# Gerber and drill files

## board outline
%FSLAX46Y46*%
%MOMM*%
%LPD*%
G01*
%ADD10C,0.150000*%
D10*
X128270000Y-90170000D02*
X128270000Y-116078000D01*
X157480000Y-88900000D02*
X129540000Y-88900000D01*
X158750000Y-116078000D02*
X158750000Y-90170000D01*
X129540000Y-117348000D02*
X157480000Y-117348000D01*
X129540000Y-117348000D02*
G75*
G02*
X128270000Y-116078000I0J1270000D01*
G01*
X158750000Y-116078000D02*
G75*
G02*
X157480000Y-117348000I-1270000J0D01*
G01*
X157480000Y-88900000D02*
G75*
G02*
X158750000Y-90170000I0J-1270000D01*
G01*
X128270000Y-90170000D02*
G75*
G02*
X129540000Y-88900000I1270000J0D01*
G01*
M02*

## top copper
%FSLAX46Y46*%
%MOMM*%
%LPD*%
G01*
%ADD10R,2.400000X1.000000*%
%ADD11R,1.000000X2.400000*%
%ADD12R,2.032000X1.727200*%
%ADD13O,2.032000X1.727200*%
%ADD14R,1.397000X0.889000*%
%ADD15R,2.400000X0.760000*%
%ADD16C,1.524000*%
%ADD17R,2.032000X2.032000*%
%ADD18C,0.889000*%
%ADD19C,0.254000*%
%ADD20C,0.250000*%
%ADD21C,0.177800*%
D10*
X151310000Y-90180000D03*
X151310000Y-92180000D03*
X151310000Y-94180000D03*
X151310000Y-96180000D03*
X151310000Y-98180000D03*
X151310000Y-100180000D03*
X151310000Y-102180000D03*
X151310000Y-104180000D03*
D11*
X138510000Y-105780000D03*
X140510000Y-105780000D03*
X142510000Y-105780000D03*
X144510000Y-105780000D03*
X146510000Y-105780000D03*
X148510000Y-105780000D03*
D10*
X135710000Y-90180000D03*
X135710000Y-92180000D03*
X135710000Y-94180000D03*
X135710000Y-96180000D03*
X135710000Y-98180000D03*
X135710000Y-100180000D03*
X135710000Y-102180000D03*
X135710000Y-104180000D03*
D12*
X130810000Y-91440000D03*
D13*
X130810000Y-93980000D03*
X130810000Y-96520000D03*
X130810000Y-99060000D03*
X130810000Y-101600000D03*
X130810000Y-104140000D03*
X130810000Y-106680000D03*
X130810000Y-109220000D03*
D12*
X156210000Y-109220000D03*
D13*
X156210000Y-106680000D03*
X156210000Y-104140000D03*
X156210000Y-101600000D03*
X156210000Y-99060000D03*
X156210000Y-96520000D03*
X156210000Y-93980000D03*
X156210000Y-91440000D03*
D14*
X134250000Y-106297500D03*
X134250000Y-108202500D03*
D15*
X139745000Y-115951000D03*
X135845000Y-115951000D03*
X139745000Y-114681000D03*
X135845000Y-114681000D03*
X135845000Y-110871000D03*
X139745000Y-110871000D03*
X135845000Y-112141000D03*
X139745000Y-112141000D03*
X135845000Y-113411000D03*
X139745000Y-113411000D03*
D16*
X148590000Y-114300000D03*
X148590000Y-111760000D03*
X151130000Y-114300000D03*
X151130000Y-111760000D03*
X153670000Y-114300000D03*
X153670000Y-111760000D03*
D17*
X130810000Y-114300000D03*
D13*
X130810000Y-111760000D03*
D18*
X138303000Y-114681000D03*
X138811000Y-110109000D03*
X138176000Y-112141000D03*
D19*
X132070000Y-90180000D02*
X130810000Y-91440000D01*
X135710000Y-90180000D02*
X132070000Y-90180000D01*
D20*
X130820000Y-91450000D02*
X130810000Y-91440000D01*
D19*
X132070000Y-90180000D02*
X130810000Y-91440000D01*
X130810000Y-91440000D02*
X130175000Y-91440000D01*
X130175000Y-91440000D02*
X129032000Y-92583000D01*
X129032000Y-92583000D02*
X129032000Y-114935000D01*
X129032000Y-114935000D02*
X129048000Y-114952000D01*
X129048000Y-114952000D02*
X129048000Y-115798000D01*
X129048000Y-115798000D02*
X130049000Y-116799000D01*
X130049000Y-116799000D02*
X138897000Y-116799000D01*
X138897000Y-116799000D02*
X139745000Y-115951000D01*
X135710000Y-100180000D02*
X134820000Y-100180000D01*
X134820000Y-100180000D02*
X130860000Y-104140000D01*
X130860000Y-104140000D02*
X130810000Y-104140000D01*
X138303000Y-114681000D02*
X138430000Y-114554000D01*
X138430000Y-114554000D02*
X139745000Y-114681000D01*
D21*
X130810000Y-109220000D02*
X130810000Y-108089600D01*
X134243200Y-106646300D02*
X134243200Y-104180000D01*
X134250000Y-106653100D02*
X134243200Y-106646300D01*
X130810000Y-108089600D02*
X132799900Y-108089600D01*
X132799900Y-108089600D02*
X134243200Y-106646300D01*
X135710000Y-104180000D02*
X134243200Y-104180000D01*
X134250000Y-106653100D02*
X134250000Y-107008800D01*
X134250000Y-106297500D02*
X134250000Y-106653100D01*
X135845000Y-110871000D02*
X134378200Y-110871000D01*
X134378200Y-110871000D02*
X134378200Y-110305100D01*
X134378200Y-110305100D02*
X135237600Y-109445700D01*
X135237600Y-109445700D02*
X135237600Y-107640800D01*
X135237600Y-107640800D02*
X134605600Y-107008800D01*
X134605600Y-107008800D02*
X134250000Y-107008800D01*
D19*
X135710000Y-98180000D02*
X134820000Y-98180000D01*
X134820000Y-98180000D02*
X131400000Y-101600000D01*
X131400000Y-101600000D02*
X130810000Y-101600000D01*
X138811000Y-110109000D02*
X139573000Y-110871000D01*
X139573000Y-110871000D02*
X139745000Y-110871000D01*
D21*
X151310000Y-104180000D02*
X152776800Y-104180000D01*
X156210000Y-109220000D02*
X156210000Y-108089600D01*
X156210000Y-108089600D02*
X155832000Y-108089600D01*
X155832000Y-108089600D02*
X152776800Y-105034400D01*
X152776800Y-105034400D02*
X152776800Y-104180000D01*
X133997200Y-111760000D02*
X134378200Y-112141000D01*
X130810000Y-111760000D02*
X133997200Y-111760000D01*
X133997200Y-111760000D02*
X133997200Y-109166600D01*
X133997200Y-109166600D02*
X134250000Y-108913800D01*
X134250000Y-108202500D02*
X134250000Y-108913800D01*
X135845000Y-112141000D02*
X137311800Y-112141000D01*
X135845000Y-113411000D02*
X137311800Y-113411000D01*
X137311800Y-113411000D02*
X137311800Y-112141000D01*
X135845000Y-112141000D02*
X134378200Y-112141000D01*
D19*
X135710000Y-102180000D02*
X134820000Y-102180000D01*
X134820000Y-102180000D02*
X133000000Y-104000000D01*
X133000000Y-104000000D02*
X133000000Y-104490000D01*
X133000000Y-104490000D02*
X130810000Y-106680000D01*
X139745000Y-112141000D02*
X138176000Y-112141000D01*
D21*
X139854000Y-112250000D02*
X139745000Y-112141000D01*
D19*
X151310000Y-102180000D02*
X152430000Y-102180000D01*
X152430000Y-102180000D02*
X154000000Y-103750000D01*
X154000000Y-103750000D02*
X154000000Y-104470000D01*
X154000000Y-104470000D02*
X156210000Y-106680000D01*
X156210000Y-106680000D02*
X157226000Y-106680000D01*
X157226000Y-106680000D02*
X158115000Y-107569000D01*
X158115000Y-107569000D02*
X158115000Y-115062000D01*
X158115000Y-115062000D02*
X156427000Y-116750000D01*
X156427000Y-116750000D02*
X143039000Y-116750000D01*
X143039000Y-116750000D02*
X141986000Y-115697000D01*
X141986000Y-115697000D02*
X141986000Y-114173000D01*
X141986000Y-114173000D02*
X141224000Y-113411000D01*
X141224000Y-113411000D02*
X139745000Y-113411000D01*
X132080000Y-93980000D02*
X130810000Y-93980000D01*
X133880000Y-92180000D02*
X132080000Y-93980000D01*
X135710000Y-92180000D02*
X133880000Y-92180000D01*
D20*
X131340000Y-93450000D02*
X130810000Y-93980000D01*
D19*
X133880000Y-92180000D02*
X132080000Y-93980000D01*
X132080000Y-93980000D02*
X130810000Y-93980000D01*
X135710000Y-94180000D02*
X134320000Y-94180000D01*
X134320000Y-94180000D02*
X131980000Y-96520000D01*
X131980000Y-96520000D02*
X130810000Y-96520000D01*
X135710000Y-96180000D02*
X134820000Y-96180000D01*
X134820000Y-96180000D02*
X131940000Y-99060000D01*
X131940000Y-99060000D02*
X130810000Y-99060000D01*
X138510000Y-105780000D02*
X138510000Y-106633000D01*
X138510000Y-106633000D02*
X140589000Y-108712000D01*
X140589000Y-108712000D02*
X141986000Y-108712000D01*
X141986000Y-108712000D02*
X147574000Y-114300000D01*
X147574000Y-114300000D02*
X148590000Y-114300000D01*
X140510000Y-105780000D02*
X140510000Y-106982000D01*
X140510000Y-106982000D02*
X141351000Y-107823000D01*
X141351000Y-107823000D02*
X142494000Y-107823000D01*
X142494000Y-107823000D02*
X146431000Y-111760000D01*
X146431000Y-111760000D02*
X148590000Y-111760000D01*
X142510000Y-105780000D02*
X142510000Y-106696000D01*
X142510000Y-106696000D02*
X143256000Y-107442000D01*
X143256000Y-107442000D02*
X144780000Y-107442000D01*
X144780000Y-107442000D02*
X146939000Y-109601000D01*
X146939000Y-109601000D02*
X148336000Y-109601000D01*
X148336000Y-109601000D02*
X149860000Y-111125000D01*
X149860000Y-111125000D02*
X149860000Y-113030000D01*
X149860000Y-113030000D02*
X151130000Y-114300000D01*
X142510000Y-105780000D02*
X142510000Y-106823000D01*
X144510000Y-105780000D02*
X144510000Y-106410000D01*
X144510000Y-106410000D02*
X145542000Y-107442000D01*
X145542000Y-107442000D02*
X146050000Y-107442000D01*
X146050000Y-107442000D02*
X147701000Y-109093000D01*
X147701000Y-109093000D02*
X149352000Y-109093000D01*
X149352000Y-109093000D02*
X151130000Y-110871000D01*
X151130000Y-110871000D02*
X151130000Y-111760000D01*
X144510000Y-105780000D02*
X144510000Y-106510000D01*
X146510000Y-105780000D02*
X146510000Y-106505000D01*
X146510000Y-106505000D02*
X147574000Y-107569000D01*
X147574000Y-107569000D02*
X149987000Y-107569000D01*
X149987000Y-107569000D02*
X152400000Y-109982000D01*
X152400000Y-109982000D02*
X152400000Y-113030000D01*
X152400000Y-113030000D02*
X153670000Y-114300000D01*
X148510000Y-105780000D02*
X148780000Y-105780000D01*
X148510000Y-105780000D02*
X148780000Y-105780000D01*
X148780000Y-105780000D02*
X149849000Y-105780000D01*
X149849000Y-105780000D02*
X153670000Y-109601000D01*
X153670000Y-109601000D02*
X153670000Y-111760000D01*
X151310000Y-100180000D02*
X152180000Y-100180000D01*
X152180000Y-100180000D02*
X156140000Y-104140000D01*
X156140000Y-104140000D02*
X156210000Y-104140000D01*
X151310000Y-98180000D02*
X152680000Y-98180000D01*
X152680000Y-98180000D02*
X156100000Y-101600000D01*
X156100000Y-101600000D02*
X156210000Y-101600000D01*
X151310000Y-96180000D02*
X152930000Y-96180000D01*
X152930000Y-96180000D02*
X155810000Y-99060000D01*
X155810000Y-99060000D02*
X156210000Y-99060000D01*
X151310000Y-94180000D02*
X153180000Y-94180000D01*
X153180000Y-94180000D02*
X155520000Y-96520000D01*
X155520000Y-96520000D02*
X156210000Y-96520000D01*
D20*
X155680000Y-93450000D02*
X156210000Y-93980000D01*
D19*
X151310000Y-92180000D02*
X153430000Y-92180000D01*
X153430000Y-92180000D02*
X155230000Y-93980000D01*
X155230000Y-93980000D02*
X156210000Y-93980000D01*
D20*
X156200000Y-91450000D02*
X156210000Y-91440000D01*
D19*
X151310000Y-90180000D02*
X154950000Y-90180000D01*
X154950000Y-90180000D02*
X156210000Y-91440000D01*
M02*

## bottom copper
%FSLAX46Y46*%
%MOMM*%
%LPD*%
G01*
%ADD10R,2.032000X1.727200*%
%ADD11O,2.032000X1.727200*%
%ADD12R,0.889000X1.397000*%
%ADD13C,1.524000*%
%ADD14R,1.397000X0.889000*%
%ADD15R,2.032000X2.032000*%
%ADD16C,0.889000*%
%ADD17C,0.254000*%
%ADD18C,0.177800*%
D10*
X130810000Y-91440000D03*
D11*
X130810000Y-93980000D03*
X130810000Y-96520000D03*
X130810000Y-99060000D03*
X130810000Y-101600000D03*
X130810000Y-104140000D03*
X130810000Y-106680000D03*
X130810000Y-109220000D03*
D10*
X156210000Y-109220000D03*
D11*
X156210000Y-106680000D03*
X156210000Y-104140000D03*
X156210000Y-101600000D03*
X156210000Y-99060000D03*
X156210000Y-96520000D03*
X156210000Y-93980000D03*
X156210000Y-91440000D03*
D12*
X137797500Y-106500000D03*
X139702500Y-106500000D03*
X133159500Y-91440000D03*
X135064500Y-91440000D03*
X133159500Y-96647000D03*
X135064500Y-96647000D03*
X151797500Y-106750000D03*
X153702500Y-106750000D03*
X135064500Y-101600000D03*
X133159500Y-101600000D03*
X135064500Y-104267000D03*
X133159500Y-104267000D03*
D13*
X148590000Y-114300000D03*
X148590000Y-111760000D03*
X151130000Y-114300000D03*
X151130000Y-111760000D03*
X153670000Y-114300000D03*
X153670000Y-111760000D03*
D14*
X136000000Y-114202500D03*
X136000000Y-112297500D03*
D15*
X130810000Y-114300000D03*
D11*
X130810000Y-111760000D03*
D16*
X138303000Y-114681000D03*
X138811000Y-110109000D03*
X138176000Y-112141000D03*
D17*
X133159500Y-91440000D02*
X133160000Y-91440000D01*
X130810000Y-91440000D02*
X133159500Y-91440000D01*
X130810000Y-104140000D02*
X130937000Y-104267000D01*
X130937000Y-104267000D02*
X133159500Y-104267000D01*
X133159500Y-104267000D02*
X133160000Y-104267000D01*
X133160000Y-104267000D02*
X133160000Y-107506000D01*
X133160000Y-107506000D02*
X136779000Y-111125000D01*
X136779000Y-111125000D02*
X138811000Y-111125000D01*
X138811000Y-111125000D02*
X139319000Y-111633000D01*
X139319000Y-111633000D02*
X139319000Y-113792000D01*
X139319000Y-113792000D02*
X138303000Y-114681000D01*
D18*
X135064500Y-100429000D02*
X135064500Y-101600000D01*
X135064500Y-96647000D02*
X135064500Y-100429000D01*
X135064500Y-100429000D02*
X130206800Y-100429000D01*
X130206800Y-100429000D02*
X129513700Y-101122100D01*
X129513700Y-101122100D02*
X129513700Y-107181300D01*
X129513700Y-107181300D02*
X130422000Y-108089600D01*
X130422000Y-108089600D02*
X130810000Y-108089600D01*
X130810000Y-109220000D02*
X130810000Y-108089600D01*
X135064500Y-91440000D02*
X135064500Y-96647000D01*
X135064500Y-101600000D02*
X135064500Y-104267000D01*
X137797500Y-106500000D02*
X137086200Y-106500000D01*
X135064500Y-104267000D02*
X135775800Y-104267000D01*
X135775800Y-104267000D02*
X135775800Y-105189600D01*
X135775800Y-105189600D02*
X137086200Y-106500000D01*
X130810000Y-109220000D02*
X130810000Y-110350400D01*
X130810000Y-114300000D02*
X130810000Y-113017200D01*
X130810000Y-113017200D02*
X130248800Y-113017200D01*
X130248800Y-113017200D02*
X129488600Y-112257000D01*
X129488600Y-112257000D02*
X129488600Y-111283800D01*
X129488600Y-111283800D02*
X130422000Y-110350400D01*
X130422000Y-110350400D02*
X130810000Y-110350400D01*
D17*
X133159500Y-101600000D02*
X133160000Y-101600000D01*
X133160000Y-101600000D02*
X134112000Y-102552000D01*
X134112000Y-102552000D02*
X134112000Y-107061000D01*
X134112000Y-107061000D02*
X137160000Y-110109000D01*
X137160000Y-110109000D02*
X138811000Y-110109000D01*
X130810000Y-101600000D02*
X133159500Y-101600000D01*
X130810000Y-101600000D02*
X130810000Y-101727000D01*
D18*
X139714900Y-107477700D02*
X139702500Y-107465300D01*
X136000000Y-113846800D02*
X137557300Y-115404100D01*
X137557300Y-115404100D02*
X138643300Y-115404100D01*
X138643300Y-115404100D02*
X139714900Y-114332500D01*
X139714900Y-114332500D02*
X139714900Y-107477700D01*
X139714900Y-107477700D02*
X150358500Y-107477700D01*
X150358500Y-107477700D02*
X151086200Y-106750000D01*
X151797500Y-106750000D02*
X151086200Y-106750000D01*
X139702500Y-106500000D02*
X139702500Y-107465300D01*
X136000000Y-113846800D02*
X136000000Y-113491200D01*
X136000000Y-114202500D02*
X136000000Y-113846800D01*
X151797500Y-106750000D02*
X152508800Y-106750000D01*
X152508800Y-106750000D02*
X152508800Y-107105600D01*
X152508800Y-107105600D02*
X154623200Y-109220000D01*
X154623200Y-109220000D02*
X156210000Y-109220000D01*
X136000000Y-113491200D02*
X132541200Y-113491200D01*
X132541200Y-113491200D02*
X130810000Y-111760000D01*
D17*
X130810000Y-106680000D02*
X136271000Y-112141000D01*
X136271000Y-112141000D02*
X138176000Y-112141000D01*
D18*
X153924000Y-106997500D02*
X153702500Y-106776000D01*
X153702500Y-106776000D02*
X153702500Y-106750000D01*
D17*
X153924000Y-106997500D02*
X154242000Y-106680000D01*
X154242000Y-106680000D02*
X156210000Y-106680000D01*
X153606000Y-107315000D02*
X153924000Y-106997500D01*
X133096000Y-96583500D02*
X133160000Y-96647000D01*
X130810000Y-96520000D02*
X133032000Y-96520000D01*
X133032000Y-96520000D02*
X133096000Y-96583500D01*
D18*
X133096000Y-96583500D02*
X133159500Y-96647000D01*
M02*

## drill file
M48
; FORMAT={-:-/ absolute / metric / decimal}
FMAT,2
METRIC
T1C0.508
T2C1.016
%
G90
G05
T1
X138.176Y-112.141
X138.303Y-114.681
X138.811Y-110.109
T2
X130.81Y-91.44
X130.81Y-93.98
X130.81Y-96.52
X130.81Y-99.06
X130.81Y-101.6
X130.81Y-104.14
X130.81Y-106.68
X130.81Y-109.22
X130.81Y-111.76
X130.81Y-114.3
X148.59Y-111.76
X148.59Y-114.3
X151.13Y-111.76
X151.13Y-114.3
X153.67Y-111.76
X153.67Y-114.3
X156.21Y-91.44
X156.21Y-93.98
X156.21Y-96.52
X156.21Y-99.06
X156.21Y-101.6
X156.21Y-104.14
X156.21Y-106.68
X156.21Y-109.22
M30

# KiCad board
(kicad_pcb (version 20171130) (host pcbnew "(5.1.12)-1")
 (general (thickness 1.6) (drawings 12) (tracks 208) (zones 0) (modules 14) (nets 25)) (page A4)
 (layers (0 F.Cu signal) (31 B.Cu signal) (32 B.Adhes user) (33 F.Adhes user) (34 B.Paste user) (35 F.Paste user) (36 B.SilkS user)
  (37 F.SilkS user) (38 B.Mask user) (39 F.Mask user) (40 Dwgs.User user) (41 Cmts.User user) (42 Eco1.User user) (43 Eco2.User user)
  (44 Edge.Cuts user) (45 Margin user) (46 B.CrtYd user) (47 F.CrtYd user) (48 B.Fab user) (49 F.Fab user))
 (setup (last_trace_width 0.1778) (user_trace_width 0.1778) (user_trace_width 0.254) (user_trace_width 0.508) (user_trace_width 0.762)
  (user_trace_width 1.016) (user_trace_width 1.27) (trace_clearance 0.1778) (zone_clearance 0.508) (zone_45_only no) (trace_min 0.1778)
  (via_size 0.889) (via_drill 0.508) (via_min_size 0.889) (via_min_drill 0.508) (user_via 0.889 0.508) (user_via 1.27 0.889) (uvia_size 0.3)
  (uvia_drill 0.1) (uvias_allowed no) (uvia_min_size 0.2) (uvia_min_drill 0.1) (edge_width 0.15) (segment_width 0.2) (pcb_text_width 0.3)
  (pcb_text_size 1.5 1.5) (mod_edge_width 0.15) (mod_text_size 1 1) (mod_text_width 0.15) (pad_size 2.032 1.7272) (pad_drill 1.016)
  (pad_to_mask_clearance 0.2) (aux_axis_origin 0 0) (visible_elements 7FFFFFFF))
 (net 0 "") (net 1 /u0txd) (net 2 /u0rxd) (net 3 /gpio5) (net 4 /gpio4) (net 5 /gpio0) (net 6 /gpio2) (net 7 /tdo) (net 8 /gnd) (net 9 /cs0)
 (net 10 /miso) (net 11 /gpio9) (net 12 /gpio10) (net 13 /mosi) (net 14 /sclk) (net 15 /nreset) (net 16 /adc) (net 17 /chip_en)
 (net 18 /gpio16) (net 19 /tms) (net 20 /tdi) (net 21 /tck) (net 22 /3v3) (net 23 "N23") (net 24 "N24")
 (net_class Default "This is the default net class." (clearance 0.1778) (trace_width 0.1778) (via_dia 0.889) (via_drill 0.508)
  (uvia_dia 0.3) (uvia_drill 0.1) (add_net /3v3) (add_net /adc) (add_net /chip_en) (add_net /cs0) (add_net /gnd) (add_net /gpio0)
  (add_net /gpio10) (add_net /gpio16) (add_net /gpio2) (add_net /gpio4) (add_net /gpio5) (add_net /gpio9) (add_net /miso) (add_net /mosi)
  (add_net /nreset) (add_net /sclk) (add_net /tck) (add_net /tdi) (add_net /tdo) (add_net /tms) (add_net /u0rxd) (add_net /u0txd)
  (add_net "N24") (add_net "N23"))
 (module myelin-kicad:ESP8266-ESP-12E (layer F.Cu) (at 143.51 93.98)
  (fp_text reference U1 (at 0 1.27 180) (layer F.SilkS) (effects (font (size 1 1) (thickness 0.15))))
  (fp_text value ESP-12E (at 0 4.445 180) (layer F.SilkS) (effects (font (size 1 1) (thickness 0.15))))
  (pad 22 smd rect (at 7.8 -3.8) (size 2.4 1) (layers F.Cu F.Paste F.Mask) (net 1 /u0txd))
  (pad 21 smd rect (at 7.8 -1.8) (size 2.4 1) (layers F.Cu F.Paste F.Mask) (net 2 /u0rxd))
  (pad 20 smd rect (at 7.8 0.2) (size 2.4 1) (layers F.Cu F.Paste F.Mask) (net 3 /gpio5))
  (pad 19 smd rect (at 7.8 2.2) (size 2.4 1) (layers F.Cu F.Paste F.Mask) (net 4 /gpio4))
  (pad 18 smd rect (at 7.8 4.2) (size 2.4 1) (layers F.Cu F.Paste F.Mask) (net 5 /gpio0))
  (pad 17 smd rect (at 7.8 6.2) (size 2.4 1) (layers F.Cu F.Paste F.Mask) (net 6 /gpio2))
  (pad 16 smd rect (at 7.8 8.2) (size 2.4 1) (layers F.Cu F.Paste F.Mask) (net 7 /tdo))
  (pad 15 smd rect (at 7.8 10.2) (size 2.4 1) (layers F.Cu F.Paste F.Mask) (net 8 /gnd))
  (pad 9 smd rect (at -5 11.8) (size 1 2.4) (layers F.Cu F.Paste F.Mask) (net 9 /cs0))
  (pad 10 smd rect (at -3 11.8) (size 1 2.4) (layers F.Cu F.Paste F.Mask) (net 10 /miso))
  (pad 11 smd rect (at -1 11.8) (size 1 2.4) (layers F.Cu F.Paste F.Mask) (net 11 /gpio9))
  (pad 12 smd rect (at 1 11.8) (size 1 2.4) (layers F.Cu F.Paste F.Mask) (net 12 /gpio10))
  (pad 13 smd rect (at 3 11.8) (size 1 2.4) (layers F.Cu F.Paste F.Mask) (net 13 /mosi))
  (pad 14 smd rect (at 5 11.8) (size 1 2.4) (layers F.Cu F.Paste F.Mask) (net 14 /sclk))
  (pad 1 smd rect (at -7.8 -3.8) (size 2.4 1) (layers F.Cu F.Paste F.Mask) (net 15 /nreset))
  (pad 2 smd rect (at -7.8 -1.8) (size 2.4 1) (layers F.Cu F.Paste F.Mask) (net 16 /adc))
  (pad 3 smd rect (at -7.8 0.2) (size 2.4 1) (layers F.Cu F.Paste F.Mask) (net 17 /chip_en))
  (pad 4 smd rect (at -7.8 2.2) (size 2.4 1) (layers F.Cu F.Paste F.Mask) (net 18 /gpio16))
  (pad 5 smd rect (at -7.8 4.2) (size 2.4 1) (layers F.Cu F.Paste F.Mask) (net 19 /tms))
  (pad 6 smd rect (at -7.8 6.2) (size 2.4 1) (layers F.Cu F.Paste F.Mask) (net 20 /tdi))
  (pad 7 smd rect (at -7.8 8.2) (size 2.4 1) (layers F.Cu F.Paste F.Mask) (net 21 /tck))
  (pad 8 smd rect (at -7.8 10.2) (size 2.4 1) (layers F.Cu F.Paste F.Mask) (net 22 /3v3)))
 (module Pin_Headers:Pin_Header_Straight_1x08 (layer F.Cu) (at 130.81 91.44)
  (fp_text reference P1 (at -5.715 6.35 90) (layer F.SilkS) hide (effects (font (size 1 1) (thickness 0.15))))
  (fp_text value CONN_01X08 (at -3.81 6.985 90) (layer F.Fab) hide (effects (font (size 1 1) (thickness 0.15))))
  (pad 1 thru_hole rect (at 0 0) (size 2.032 1.7272) (drill 1.016) (layers *.Cu *.Mask F.SilkS) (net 15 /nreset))
  (pad 2 thru_hole oval (at 0 2.54) (size 2.032 1.7272) (drill 1.016) (layers *.Cu *.Mask F.SilkS) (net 16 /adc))
  (pad 3 thru_hole oval (at 0 5.08) (size 2.032 1.7272) (drill 1.016) (layers *.Cu *.Mask F.SilkS) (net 17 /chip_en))
  (pad 4 thru_hole oval (at 0 7.62) (size 2.032 1.7272) (drill 1.016) (layers *.Cu *.Mask F.SilkS) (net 18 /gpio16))
  (pad 5 thru_hole oval (at 0 10.16) (size 2.032 1.7272) (drill 1.016) (layers *.Cu *.Mask F.SilkS) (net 19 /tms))
  (pad 6 thru_hole oval (at 0 12.7) (size 2.032 1.7272) (drill 1.016) (layers *.Cu *.Mask F.SilkS) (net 20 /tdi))
  (pad 7 thru_hole oval (at 0 15.24) (size 2.032 1.7272) (drill 1.016) (layers *.Cu *.Mask F.SilkS) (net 21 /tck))
  (pad 8 thru_hole oval (at 0 17.78) (size 2.032 1.7272) (drill 1.016) (layers *.Cu *.Mask F.SilkS) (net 22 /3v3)))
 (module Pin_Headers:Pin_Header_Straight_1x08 (layer F.Cu) (at 156.21 109.22 180)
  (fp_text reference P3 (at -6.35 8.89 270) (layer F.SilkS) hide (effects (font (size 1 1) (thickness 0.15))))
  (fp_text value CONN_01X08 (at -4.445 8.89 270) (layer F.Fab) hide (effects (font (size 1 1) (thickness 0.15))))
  (pad 1 thru_hole rect (at 0 0 180) (size 2.032 1.7272) (drill 1.016) (layers *.Cu *.Mask F.SilkS) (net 8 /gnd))
  (pad 2 thru_hole oval (at 0 2.54 180) (size 2.032 1.7272) (drill 1.016) (layers *.Cu *.Mask F.SilkS) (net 7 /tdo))
  (pad 3 thru_hole oval (at 0 5.08 180) (size 2.032 1.7272) (drill 1.016) (layers *.Cu *.Mask F.SilkS) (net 6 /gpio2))
  (pad 4 thru_hole oval (at 0 7.62 180) (size 2.032 1.7272) (drill 1.016) (layers *.Cu *.Mask F.SilkS) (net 5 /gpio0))
  (pad 5 thru_hole oval (at 0 10.16 180) (size 2.032 1.7272) (drill 1.016) (layers *.Cu *.Mask F.SilkS) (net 4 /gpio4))
  (pad 6 thru_hole oval (at 0 12.7 180) (size 2.032 1.7272) (drill 1.016) (layers *.Cu *.Mask F.SilkS) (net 3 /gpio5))
  (pad 7 thru_hole oval (at 0 15.24 180) (size 2.032 1.7272) (drill 1.016) (layers *.Cu *.Mask F.SilkS) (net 2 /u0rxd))
  (pad 8 thru_hole oval (at 0 17.78 180) (size 2.032 1.7272) (drill 1.016) (layers *.Cu *.Mask F.SilkS) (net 1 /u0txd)))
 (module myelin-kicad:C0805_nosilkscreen (layer B.Cu) (at 138.75 106.5)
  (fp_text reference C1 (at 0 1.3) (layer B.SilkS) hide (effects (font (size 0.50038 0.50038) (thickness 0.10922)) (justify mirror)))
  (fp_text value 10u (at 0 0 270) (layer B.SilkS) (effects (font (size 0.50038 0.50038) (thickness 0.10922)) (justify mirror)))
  (pad 1 smd rect (at -0.9525 0) (size 0.889 1.397) (layers B.Cu B.Paste B.Mask) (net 22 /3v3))
  (pad 2 smd rect (at 0.9525 0) (size 0.889 1.397) (layers B.Cu B.Paste B.Mask) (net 8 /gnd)))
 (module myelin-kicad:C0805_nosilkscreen (layer F.Cu) (at 134.25 107.25 270)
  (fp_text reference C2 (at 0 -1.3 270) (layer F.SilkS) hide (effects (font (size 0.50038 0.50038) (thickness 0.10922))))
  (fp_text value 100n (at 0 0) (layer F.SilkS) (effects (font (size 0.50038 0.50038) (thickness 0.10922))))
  (pad 1 smd rect (at -0.9525 0 270) (size 0.889 1.397) (layers F.Cu F.Paste F.Mask) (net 22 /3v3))
  (pad 2 smd rect (at 0.9525 0 270) (size 0.889 1.397) (layers F.Cu F.Paste F.Mask) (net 8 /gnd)))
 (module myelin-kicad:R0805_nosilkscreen (layer B.Cu) (at 134.112 91.44)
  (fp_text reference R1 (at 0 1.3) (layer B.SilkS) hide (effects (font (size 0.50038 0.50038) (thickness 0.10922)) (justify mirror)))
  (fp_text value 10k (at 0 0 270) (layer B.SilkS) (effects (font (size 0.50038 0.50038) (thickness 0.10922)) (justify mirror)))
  (pad 1 smd rect (at -0.9525 0) (size 0.889 1.397) (layers B.Cu B.Paste B.Mask) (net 15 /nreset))
  (pad 2 smd rect (at 0.9525 0) (size 0.889 1.397) (layers B.Cu B.Paste B.Mask) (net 22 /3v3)))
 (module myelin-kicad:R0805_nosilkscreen (layer B.Cu) (at 134.112 96.647)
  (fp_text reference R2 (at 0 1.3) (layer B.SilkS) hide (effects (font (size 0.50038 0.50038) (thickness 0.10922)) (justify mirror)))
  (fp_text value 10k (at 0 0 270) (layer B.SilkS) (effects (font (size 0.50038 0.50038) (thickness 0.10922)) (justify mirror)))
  (pad 1 smd rect (at -0.9525 0) (size 0.889 1.397) (layers B.Cu B.Paste B.Mask) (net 17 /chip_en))
  (pad 2 smd rect (at 0.9525 0) (size 0.889 1.397) (layers B.Cu B.Paste B.Mask) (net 22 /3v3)))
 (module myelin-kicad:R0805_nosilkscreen (layer B.Cu) (at 152.75 106.75)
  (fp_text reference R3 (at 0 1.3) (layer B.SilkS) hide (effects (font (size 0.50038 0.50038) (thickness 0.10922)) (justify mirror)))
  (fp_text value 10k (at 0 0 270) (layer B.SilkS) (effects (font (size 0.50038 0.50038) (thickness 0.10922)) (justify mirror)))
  (pad 1 smd rect (at -0.9525 0) (size 0.889 1.397) (layers B.Cu B.Paste B.Mask) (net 8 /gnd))
  (pad 2 smd rect (at 0.9525 0) (size 0.889 1.397) (layers B.Cu B.Paste B.Mask) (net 7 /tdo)))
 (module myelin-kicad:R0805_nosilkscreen (layer B.Cu) (at 134.112 101.6 180)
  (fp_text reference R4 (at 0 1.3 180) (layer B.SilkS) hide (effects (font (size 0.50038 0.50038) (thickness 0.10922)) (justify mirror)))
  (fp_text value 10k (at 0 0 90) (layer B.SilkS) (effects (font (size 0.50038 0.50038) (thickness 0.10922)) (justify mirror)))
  (pad 1 smd rect (at -0.9525 0 180) (size 0.889 1.397) (layers B.Cu B.Paste B.Mask) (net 22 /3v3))
  (pad 2 smd rect (at 0.9525 0 180) (size 0.889 1.397) (layers B.Cu B.Paste B.Mask) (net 19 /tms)))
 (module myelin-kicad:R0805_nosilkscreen (layer B.Cu) (at 134.112 104.267 180)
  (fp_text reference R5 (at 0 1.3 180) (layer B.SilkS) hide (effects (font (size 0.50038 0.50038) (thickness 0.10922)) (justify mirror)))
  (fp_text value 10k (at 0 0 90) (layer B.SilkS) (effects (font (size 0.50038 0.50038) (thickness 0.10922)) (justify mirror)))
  (pad 1 smd rect (at -0.9525 0 180) (size 0.889 1.397) (layers B.Cu B.Paste B.Mask) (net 22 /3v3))
  (pad 2 smd rect (at 0.9525 0 180) (size 0.889 1.397) (layers B.Cu B.Paste B.Mask) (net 20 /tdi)))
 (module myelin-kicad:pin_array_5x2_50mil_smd (layer F.Cu) (at 137.795 113.411 270)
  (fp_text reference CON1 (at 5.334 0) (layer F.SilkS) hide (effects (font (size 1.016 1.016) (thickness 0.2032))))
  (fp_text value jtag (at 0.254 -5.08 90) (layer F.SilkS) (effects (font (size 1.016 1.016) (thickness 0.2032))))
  (pad 10 smd rect (at 2.54 -1.95 270) (size 0.76 2.4) (layers F.Cu F.Paste F.Mask) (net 15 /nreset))
  (pad 9 smd rect (at 2.54 1.95 270) (size 0.76 2.4) (layers F.Cu F.Paste F.Mask) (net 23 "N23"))
  (pad 8 smd rect (at 1.27 -1.95 270) (size 0.76 2.4) (layers F.Cu F.Paste F.Mask) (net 20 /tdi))
  (pad 7 smd rect (at 1.27 1.95 270) (size 0.76 2.4) (layers F.Cu F.Paste F.Mask) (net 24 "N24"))
  (pad 1 smd rect (at -2.54 1.95 270) (size 0.76 2.4) (layers F.Cu F.Paste F.Mask) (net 22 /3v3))
  (pad 2 smd rect (at -2.54 -1.95 270) (size 0.76 2.4) (layers F.Cu F.Paste F.Mask) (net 19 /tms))
  (pad 3 smd rect (at -1.27 1.95 270) (size 0.76 2.4) (layers F.Cu F.Paste F.Mask) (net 8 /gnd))
  (pad 4 smd rect (at -1.27 -1.95 270) (size 0.76 2.4) (layers F.Cu F.Paste F.Mask) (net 21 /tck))
  (pad 5 smd rect (at 0 1.95 270) (size 0.76 2.4) (layers F.Cu F.Paste F.Mask) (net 8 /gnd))
  (pad 6 smd rect (at 0 -1.95 270) (size 0.76 2.4) (layers F.Cu F.Paste F.Mask) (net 7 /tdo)))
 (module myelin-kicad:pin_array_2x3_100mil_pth (layer F.Cu) (at 151.13 113.03)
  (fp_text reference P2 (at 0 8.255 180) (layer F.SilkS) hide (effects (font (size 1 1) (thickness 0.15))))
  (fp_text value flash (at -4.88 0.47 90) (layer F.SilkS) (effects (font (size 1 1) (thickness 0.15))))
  (pad 1 thru_hole circle (at -2.54 1.27) (size 1.524 1.524) (drill 1.016) (layers *.Cu *.Mask F.SilkS) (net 9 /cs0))
  (pad 2 thru_hole circle (at -2.54 -1.27) (size 1.524 1.524) (drill 1.016) (layers *.Cu *.Mask F.SilkS) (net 10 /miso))
  (pad 3 thru_hole circle (at 0 1.27) (size 1.524 1.524) (drill 1.016) (layers *.Cu *.Mask F.SilkS) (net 11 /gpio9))
  (pad 4 thru_hole circle (at 0 -1.27) (size 1.524 1.524) (drill 1.016) (layers *.Cu *.Mask F.SilkS) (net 12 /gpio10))
  (pad 5 thru_hole circle (at 2.54 1.27) (size 1.524 1.524) (drill 1.016) (layers *.Cu *.Mask F.SilkS) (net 13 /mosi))
  (pad 6 thru_hole circle (at 2.54 -1.27) (size 1.524 1.524) (drill 1.016) (layers *.Cu *.Mask F.SilkS) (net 14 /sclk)))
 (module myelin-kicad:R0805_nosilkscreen (layer B.Cu) (at 136 113.25 90)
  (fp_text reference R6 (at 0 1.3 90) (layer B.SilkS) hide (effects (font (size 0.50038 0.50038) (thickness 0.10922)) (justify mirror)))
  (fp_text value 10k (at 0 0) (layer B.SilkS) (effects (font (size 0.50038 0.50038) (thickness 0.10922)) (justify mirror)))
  (pad 1 smd rect (at -0.9525 0 90) (size 0.889 1.397) (layers B.Cu B.Paste B.Mask) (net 8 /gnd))
  (pad 2 smd rect (at 0.9525 0 90) (size 0.889 1.397) (layers B.Cu B.Paste B.Mask) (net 21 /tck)))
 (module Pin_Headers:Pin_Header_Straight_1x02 (layer F.Cu) (at 130.81 114.3 180)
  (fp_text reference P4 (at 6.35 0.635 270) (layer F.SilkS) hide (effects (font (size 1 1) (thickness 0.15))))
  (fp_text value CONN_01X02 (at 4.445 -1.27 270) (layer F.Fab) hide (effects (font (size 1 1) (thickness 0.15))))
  (pad 1 thru_hole rect (at 0 0 180) (size 2.032 2.032) (drill 1.016) (layers *.Cu *.Mask F.SilkS) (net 22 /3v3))
  (pad 2 thru_hole oval (at 0 2.54 180) (size 2.032 1.7272) (drill 1.016) (layers *.Cu *.Mask F.SilkS) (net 8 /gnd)))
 (gr_line (start 128.27 90.17) (end 128.27 116.078) (angle 90) (layer Edge.Cuts) (width 0.15))
 (gr_line (start 157.48 88.9) (end 129.54 88.9) (angle 90) (layer Edge.Cuts) (width 0.15))
 (gr_line (start 158.75 116.078) (end 158.75 90.17) (angle 90) (layer Edge.Cuts) (width 0.15))
 (gr_line (start 129.54 117.348) (end 157.48 117.348) (angle 90) (layer Edge.Cuts) (width 0.15))
 (gr_arc (start 129.54 116.078) (end 129.54 117.348) (angle 90) (layer Edge.Cuts) (width 0.15))
 (gr_arc (start 157.48 116.078) (end 158.75 116.078) (angle 90) (layer Edge.Cuts) (width 0.15))
 (gr_arc (start 157.48 90.17) (end 157.48 88.9) (angle 90) (layer Edge.Cuts) (width 0.15))
 (gr_arc (start 129.54 90.17) (end 128.27 90.17) (angle 90) (layer Edge.Cuts) (width 0.15))
 (segment (start 133.1595 91.44) (end 133.16 91.44) (width 0.254) (layer B.Cu) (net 15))
 (segment (start 130.81 91.44) (end 133.1595 91.44) (width 0.254) (layer B.Cu) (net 15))
 (segment (start 132.07 90.18) (end 130.81 91.44) (width 0.254) (layer F.Cu) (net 15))
 (segment (start 135.71 90.18) (end 132.07 90.18) (width 0.254) (layer F.Cu) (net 15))
 (segment (start 130.82 91.45) (end 130.81 91.44) (width 0.25) (layer F.Cu) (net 15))
 (segment (start 132.07 90.18) (end 130.81 91.44) (width 0.254) (layer F.Cu) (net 15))
 (segment (start 130.81 91.44) (end 130.175 91.44) (width 0.254) (layer F.Cu) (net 15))
 (segment (start 130.175 91.44) (end 129.032 92.583) (width 0.254) (layer F.Cu) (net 15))
 (segment (start 129.032 92.583) (end 129.032 114.935) (width 0.254) (layer F.Cu) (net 15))
 (segment (start 129.032 114.935) (end 129.048 114.952) (width 0.254) (layer F.Cu) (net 15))
 (segment (start 129.048 114.952) (end 129.048 115.798) (width 0.254) (layer F.Cu) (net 15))
 (segment (start 129.048 115.798) (end 130.049 116.799) (width 0.254) (layer F.Cu) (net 15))
 (segment (start 130.049 116.799) (end 138.897 116.799) (width 0.254) (layer F.Cu) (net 15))
 (segment (start 138.897 116.799) (end 139.745 115.951) (width 0.254) (layer F.Cu) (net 15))
 (segment (start 130.81 104.14) (end 130.937 104.267) (width 0.254) (layer B.Cu) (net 20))
 (segment (start 130.937 104.267) (end 133.1595 104.267) (width 0.254) (layer B.Cu) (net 20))
 (segment (start 135.71 100.18) (end 134.82 100.18) (width 0.254) (layer F.Cu) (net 20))
 (segment (start 134.82 100.18) (end 130.86 104.14) (width 0.254) (layer F.Cu) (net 20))
 (segment (start 130.86 104.14) (end 130.81 104.14) (width 0.254) (layer F.Cu) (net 20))
 (segment (start 133.1595 104.267) (end 133.16 104.267) (width 0.254) (layer B.Cu) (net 20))
 (segment (start 133.16 104.267) (end 133.16 107.506) (width 0.254) (layer B.Cu) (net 20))
 (segment (start 133.16 107.506) (end 136.779 111.125) (width 0.254) (layer B.Cu) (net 20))
 (segment (start 136.779 111.125) (end 138.811 111.125) (width 0.254) (layer B.Cu) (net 20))
 (segment (start 138.811 111.125) (end 139.319 111.633) (width 0.254) (layer B.Cu) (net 20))
 (segment (start 139.319 111.633) (end 139.319 113.792) (width 0.254) (layer B.Cu) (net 20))
 (segment (start 139.319 113.792) (end 138.303 114.681) (width 0.254) (layer B.Cu) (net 20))
 (segment (start 138.303 114.681) (end 138.43 114.554) (width 0.254) (layer F.Cu) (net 20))
 (segment (start 138.43 114.554) (end 139.745 114.681) (width 0.254) (layer F.Cu) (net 20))
 (via (at 138.303 114.681) (size 0.889) (layers F.Cu B.Cu) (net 20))
 (segment (start 130.81 109.22) (end 130.81 108.0896) (width 0.1778) (layer F.Cu) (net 22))
 (segment (start 134.2432 106.6463) (end 134.2432 104.18) (width 0.1778) (layer F.Cu) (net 22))
 (segment (start 134.25 106.6531) (end 134.2432 106.6463) (width 0.1778) (layer F.Cu) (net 22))
 (segment (start 130.81 108.0896) (end 132.7999 108.0896) (width 0.1778) (layer F.Cu) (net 22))
 (segment (start 132.7999 108.0896) (end 134.2432 106.6463) (width 0.1778) (layer F.Cu) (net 22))
 (segment (start 135.0645 100.429) (end 135.0645 101.6) (width 0.1778) (layer B.Cu) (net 22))
 (segment (start 135.0645 96.647) (end 135.0645 100.429) (width 0.1778) (layer B.Cu) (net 22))
 (segment (start 135.0645 100.429) (end 130.2068 100.429) (width 0.1778) (layer B.Cu) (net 22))
 (segment (start 130.2068 100.429) (end 129.5137 101.1221) (width 0.1778) (layer B.Cu) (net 22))
 (segment (start 129.5137 101.1221) (end 129.5137 107.1813) (width 0.1778) (layer B.Cu) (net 22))
 (segment (start 129.5137 107.1813) (end 130.422 108.0896) (width 0.1778) (layer B.Cu) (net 22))
 (segment (start 130.422 108.0896) (end 130.81 108.0896) (width 0.1778) (layer B.Cu) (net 22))
 (segment (start 130.81 109.22) (end 130.81 108.0896) (width 0.1778) (layer B.Cu) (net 22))
 (segment (start 135.71 104.18) (end 134.2432 104.18) (width 0.1778) (layer F.Cu) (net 22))
 (segment (start 134.25 106.6531) (end 134.25 107.0088) (width 0.1778) (layer F.Cu) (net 22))
 (segment (start 134.25 106.2975) (end 134.25 106.6531) (width 0.1778) (layer F.Cu) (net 22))
 (segment (start 135.0645 91.44) (end 135.0645 96.647) (width 0.1778) (layer B.Cu) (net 22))
 (segment (start 135.0645 101.6) (end 135.0645 104.267) (width 0.1778) (layer B.Cu) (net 22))
 (segment (start 137.7975 106.5) (end 137.0862 106.5) (width 0.1778) (layer B.Cu) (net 22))
 (segment (start 135.0645 104.267) (end 135.7758 104.267) (width 0.1778) (layer B.Cu) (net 22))
 (segment (start 135.7758 104.267) (end 135.7758 105.1896) (width 0.1778) (layer B.Cu) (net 22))
 (segment (start 135.7758 105.1896) (end 137.0862 106.5) (width 0.1778) (layer B.Cu) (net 22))
 (segment (start 135.845 110.871) (end 134.3782 110.871) (width 0.1778) (layer F.Cu) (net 22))
 (segment (start 134.3782 110.871) (end 134.3782 110.3051) (width 0.1778) (layer F.Cu) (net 22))
 (segment (start 134.3782 110.3051) (end 135.2376 109.4457) (width 0.1778) (layer F.Cu) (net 22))
 (segment (start 135.2376 109.4457) (end 135.2376 107.6408) (width 0.1778) (layer F.Cu) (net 22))
 (segment (start 135.2376 107.6408) (end 134.6056 107.0088) (width 0.1778) (layer F.Cu) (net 22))
 (segment (start 134.6056 107.0088) (end 134.25 107.0088) (width 0.1778) (layer F.Cu) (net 22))
 (segment (start 130.81 109.22) (end 130.81 110.3504) (width 0.1778) (layer B.Cu) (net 22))
 (segment (start 130.81 114.3) (end 130.81 113.0172) (width 0.1778) (layer B.Cu) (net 22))
 (segment (start 130.81 113.0172) (end 130.2488 113.0172) (width 0.1778) (layer B.Cu) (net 22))
 (segment (start 130.2488 113.0172) (end 129.4886 112.257) (width 0.1778) (layer B.Cu) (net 22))
 (segment (start 129.4886 112.257) (end 129.4886 111.2838) (width 0.1778) (layer B.Cu) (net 22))
 (segment (start 129.4886 111.2838) (end 130.422 110.3504) (width 0.1778) (layer B.Cu) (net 22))
 (segment (start 130.422 110.3504) (end 130.81 110.3504) (width 0.1778) (layer B.Cu) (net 22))
 (segment (start 133.1595 101.6) (end 133.16 101.6) (width 0.254) (layer B.Cu) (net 19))
 (segment (start 133.16 101.6) (end 134.112 102.552) (width 0.254) (layer B.Cu) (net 19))
 (segment (start 134.112 102.552) (end 134.112 107.061) (width 0.254) (layer B.Cu) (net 19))
 (segment (start 134.112 107.061) (end 137.16 110.109) (width 0.254) (layer B.Cu) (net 19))
 (segment (start 137.16 110.109) (end 138.811 110.109) (width 0.254) (layer B.Cu) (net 19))
 (segment (start 130.81 101.6) (end 133.1595 101.6) (width 0.254) (layer B.Cu) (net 19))
 (segment (start 135.71 98.18) (end 134.82 98.18) (width 0.254) (layer F.Cu) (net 19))
 (segment (start 134.82 98.18) (end 131.4 101.6) (width 0.254) (layer F.Cu) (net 19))
 (segment (start 131.4 101.6) (end 130.81 101.6) (width 0.254) (layer F.Cu) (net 19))
 (segment (start 138.811 110.109) (end 139.573 110.871) (width 0.254) (layer F.Cu) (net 19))
 (segment (start 139.573 110.871) (end 139.745 110.871) (width 0.254) (layer F.Cu) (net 19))
 (segment (start 130.81 101.6) (end 130.81 101.727) (width 0.254) (layer B.Cu) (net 19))
 (via (at 138.811 110.109) (size 0.889) (layers F.Cu B.Cu) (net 19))
 (segment (start 151.31 104.18) (end 152.7768 104.18) (width 0.1778) (layer F.Cu) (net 8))
 (segment (start 156.21 109.22) (end 156.21 108.0896) (width 0.1778) (layer F.Cu) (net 8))
 (segment (start 156.21 108.0896) (end 155.832 108.0896) (width 0.1778) (layer F.Cu) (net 8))
 (segment (start 155.832 108.0896) (end 152.7768 105.0344) (width 0.1778) (layer F.Cu) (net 8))
 (segment (start 152.7768 105.0344) (end 152.7768 104.18) (width 0.1778) (layer F.Cu) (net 8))
 (segment (start 139.7149 107.4777) (end 139.7025 107.4653) (width 0.1778) (layer B.Cu) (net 8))
 (segment (start 136 113.8468) (end 137.5573 115.4041) (width 0.1778) (layer B.Cu) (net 8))
 (segment (start 137.5573 115.4041) (end 138.6433 115.4041) (width 0.1778) (layer B.Cu) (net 8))
 (segment (start 138.6433 115.4041) (end 139.7149 114.3325) (width 0.1778) (layer B.Cu) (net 8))
 (segment (start 139.7149 114.3325) (end 139.7149 107.4777) (width 0.1778) (layer B.Cu) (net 8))
 (segment (start 139.7149 107.4777) (end 150.3585 107.4777) (width 0.1778) (layer B.Cu) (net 8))
 (segment (start 150.3585 107.4777) (end 151.0862 106.75) (width 0.1778) (layer B.Cu) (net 8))
 (segment (start 151.7975 106.75) (end 151.0862 106.75) (width 0.1778) (layer B.Cu) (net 8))
 (segment (start 139.7025 106.5) (end 139.7025 107.4653) (width 0.1778) (layer B.Cu) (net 8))
 (segment (start 136 113.8468) (end 136 113.4912) (width 0.1778) (layer B.Cu) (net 8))
 (segment (start 136 114.2025) (end 136 113.8468) (width 0.1778) (layer B.Cu) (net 8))
 (segment (start 151.7975 106.75) (end 152.5088 106.75) (width 0.1778) (layer B.Cu) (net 8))
 (segment (start 152.5088 106.75) (end 152.5088 107.1056) (width 0.1778) (layer B.Cu) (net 8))
 (segment (start 152.5088 107.1056) (end 154.6232 109.22) (width 0.1778) (layer B.Cu) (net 8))
 (segment (start 154.6232 109.22) (end 156.21 109.22) (width 0.1778) (layer B.Cu) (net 8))
 (segment (start 136 113.4912) (end 132.5412 113.4912) (width 0.1778) (layer B.Cu) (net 8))
 (segment (start 132.5412 113.4912) (end 130.81 111.76) (width 0.1778) (layer B.Cu) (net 8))
 (segment (start 133.9972 111.76) (end 134.3782 112.141) (width 0.1778) (layer F.Cu) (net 8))
 (segment (start 130.81 111.76) (end 133.9972 111.76) (width 0.1778) (layer F.Cu) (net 8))
 (segment (start 133.9972 111.76) (end 133.9972 109.1666) (width 0.1778) (layer F.Cu) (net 8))
 (segment (start 133.9972 109.1666) (end 134.25 108.9138) (width 0.1778) (layer F.Cu) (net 8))
 (segment (start 134.25 108.2025) (end 134.25 108.9138) (width 0.1778) (layer F.Cu) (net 8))
 (segment (start 135.845 112.141) (end 137.3118 112.141) (width 0.1778) (layer F.Cu) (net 8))
 (segment (start 135.845 113.411) (end 137.3118 113.411) (width 0.1778) (layer F.Cu) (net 8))
 (segment (start 137.3118 113.411) (end 137.3118 112.141) (width 0.1778) (layer F.Cu) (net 8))
 (segment (start 135.845 112.141) (end 134.3782 112.141) (width 0.1778) (layer F.Cu) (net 8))
 (segment (start 130.81 106.68) (end 136.271 112.141) (width 0.254) (layer B.Cu) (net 21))
 (segment (start 136.271 112.141) (end 138.176 112.141) (width 0.254) (layer B.Cu) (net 21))
 (segment (start 135.71 102.18) (end 134.82 102.18) (width 0.254) (layer F.Cu) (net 21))
 (segment (start 134.82 102.18) (end 133 104) (width 0.254) (layer F.Cu) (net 21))
 (segment (start 133 104) (end 133 104.49) (width 0.254) (layer F.Cu) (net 21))
 (segment (start 133 104.49) (end 130.81 106.68) (width 0.254) (layer F.Cu) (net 21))
 (segment (start 139.745 112.141) (end 138.176 112.141) (width 0.254) (layer F.Cu) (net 21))
 (segment (start 139.854 112.25) (end 139.745 112.141) (width 0.1778) (layer F.Cu) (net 21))
 (via (at 138.176 112.141) (size 0.889) (layers F.Cu B.Cu) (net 21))
 (segment (start 153.924 106.9975) (end 153.7025 106.776) (width 0.1778) (layer B.Cu) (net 7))
 (segment (start 153.7025 106.776) (end 153.7025 106.75) (width 0.1778) (layer B.Cu) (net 7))
 (segment (start 153.924 106.9975) (end 154.242 106.68) (width 0.254) (layer B.Cu) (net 7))
 (segment (start 154.242 106.68) (end 156.21 106.68) (width 0.254) (layer B.Cu) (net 7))
 (segment (start 153.606 107.315) (end 153.924 106.9975) (width 0.254) (layer B.Cu) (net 7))
 (segment (start 151.31 102.18) (end 152.43 102.18) (width 0.254) (layer F.Cu) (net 7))
 (segment (start 152.43 102.18) (end 154 103.75) (width 0.254) (layer F.Cu) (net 7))
 (segment (start 154 103.75) (end 154 104.47) (width 0.254) (layer F.Cu) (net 7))
 (segment (start 154 104.47) (end 156.21 106.68) (width 0.254) (layer F.Cu) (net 7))
 (segment (start 156.21 106.68) (end 157.226 106.68) (width 0.254) (layer F.Cu) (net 7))
 (segment (start 157.226 106.68) (end 158.115 107.569) (width 0.254) (layer F.Cu) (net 7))
 (segment (start 158.115 107.569) (end 158.115 115.062) (width 0.254) (layer F.Cu) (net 7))
 (segment (start 158.115 115.062) (end 156.427 116.75) (width 0.254) (layer F.Cu) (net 7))
 (segment (start 156.427 116.75) (end 143.039 116.75) (width 0.254) (layer F.Cu) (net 7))
 (segment (start 143.039 116.75) (end 141.986 115.697) (width 0.254) (layer F.Cu) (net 7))
 (segment (start 141.986 115.697) (end 141.986 114.173) (width 0.254) (layer F.Cu) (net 7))
 (segment (start 141.986 114.173) (end 141.224 113.411) (width 0.254) (layer F.Cu) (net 7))
 (segment (start 141.224 113.411) (end 139.745 113.411) (width 0.254) (layer F.Cu) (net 7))
 (segment (start 132.08 93.98) (end 130.81 93.98) (width 0.254) (layer F.Cu) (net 16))
 (segment (start 133.88 92.18) (end 132.08 93.98) (width 0.254) (layer F.Cu) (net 16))
 (segment (start 135.71 92.18) (end 133.88 92.18) (width 0.254) (layer F.Cu) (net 16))
 (segment (start 131.34 93.45) (end 130.81 93.98) (width 0.25) (layer F.Cu) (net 16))
 (segment (start 133.88 92.18) (end 132.08 93.98) (width 0.254) (layer F.Cu) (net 16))
 (segment (start 132.08 93.98) (end 130.81 93.98) (width 0.254) (layer F.Cu) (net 16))
 (segment (start 133.096 96.5835) (end 133.16 96.647) (width 0.254) (layer B.Cu) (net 17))
 (segment (start 130.81 96.52) (end 133.032 96.52) (width 0.254) (layer B.Cu) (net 17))
 (segment (start 133.032 96.52) (end 133.096 96.5835) (width 0.254) (layer B.Cu) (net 17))
 (segment (start 133.096 96.5835) (end 133.1595 96.647) (width 0.1778) (layer B.Cu) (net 17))
 (segment (start 135.71 94.18) (end 134.32 94.18) (width 0.254) (layer F.Cu) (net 17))
 (segment (start 134.32 94.18) (end 131.98 96.52) (width 0.254) (layer F.Cu) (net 17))
 (segment (start 131.98 96.52) (end 130.81 96.52) (width 0.254) (layer F.Cu) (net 17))
 (segment (start 135.71 96.18) (end 134.82 96.18) (width 0.254) (layer F.Cu) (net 18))
 (segment (start 134.82 96.18) (end 131.94 99.06) (width 0.254) (layer F.Cu) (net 18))
 (segment (start 131.94 99.06) (end 130.81 99.06) (width 0.254) (layer F.Cu) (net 18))
 (segment (start 138.51 105.78) (end 138.51 106.633) (width 0.254) (layer F.Cu) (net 9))
 (segment (start 138.51 106.633) (end 140.589 108.712) (width 0.254) (layer F.Cu) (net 9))
 (segment (start 140.589 108.712) (end 141.986 108.712) (width 0.254) (layer F.Cu) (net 9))
 (segment (start 141.986 108.712) (end 147.574 114.3) (width 0.254) (layer F.Cu) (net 9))
 (segment (start 147.574 114.3) (end 148.59 114.3) (width 0.254) (layer F.Cu) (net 9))
 (segment (start 140.51 105.78) (end 140.51 106.982) (width 0.254) (layer F.Cu) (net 10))
 (segment (start 140.51 106.982) (end 141.351 107.823) (width 0.254) (layer F.Cu) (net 10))
 (segment (start 141.351 107.823) (end 142.494 107.823) (width 0.254) (layer F.Cu) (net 10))
 (segment (start 142.494 107.823) (end 146.431 111.76) (width 0.254) (layer F.Cu) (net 10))
 (segment (start 146.431 111.76) (end 148.59 111.76) (width 0.254) (layer F.Cu) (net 10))
 (segment (start 142.51 105.78) (end 142.51 106.696) (width 0.254) (layer F.Cu) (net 11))
 (segment (start 142.51 106.696) (end 143.256 107.442) (width 0.254) (layer F.Cu) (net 11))
 (segment (start 143.256 107.442) (end 144.78 107.442) (width 0.254) (layer F.Cu) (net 11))
 (segment (start 144.78 107.442) (end 146.939 109.601) (width 0.254) (layer F.Cu) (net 11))
 (segment (start 146.939 109.601) (end 148.336 109.601) (width 0.254) (layer F.Cu) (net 11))
 (segment (start 148.336 109.601) (end 149.86 111.125) (width 0.254) (layer F.Cu) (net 11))
 (segment (start 149.86 111.125) (end 149.86 113.03) (width 0.254) (layer F.Cu) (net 11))
 (segment (start 149.86 113.03) (end 151.13 114.3) (width 0.254) (layer F.Cu) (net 11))
 (segment (start 142.51 105.78) (end 142.51 106.823) (width 0.254) (layer F.Cu) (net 11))
 (segment (start 144.51 105.78) (end 144.51 106.41) (width 0.254) (layer F.Cu) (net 12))
 (segment (start 144.51 106.41) (end 145.542 107.442) (width 0.254) (layer F.Cu) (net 12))
 (segment (start 145.542 107.442) (end 146.05 107.442) (width 0.254) (layer F.Cu) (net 12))
 (segment (start 146.05 107.442) (end 147.701 109.093) (width 0.254) (layer F.Cu) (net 12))
 (segment (start 147.701 109.093) (end 149.352 109.093) (width 0.254) (layer F.Cu) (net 12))
 (segment (start 149.352 109.093) (end 151.13 110.871) (width 0.254) (layer F.Cu) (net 12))
 (segment (start 151.13 110.871) (end 151.13 111.76) (width 0.254) (layer F.Cu) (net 12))
 (segment (start 144.51 105.78) (end 144.51 106.51) (width 0.254) (layer F.Cu) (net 12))
 (segment (start 146.51 105.78) (end 146.51 106.505) (width 0.254) (layer F.Cu) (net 13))
 (segment (start 146.51 106.505) (end 147.574 107.569) (width 0.254) (layer F.Cu) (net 13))
 (segment (start 147.574 107.569) (end 149.987 107.569) (width 0.254) (layer F.Cu) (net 13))
 (segment (start 149.987 107.569) (end 152.4 109.982) (width 0.254) (layer F.Cu) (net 13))
 (segment (start 152.4 109.982) (end 152.4 113.03) (width 0.254) (layer F.Cu) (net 13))
 (segment (start 152.4 113.03) (end 153.67 114.3) (width 0.254) (layer F.Cu) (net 13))
 (segment (start 148.51 105.78) (end 148.78 105.78) (width 0.254) (layer F.Cu) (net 14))
 (segment (start 148.51 105.78) (end 148.78 105.78) (width 0.254) (layer F.Cu) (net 14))
 (segment (start 148.78 105.78) (end 149.849 105.78) (width 0.254) (layer F.Cu) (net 14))
 (segment (start 149.849 105.78) (end 153.67 109.601) (width 0.254) (layer F.Cu) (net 14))
 (segment (start 153.67 109.601) (end 153.67 111.76) (width 0.254) (layer F.Cu) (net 14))
 (segment (start 151.31 100.18) (end 152.18 100.18) (width 0.254) (layer F.Cu) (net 6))
 (segment (start 152.18 100.18) (end 156.14 104.14) (width 0.254) (layer F.Cu) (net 6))
 (segment (start 156.14 104.14) (end 156.21 104.14) (width 0.254) (layer F.Cu) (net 6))
 (segment (start 151.31 98.18) (end 152.68 98.18) (width 0.254) (layer F.Cu) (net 5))
 (segment (start 152.68 98.18) (end 156.1 101.6) (width 0.254) (layer F.Cu) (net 5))
 (segment (start 156.1 101.6) (end 156.21 101.6) (width 0.254) (layer F.Cu) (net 5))
 (segment (start 151.31 96.18) (end 152.93 96.18) (width 0.254) (layer F.Cu) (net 4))
 (segment (start 152.93 96.18) (end 155.81 99.06) (width 0.254) (layer F.Cu) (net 4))
 (segment (start 155.81 99.06) (end 156.21 99.06) (width 0.254) (layer F.Cu) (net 4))
 (segment (start 151.31 94.18) (end 153.18 94.18) (width 0.254) (layer F.Cu) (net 3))
 (segment (start 153.18 94.18) (end 155.52 96.52) (width 0.254) (layer F.Cu) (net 3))
 (segment (start 155.52 96.52) (end 156.21 96.52) (width 0.254) (layer F.Cu) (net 3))
 (segment (start 155.68 93.45) (end 156.21 93.98) (width 0.25) (layer F.Cu) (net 2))
 (segment (start 151.31 92.18) (end 153.43 92.18) (width 0.254) (layer F.Cu) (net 2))
 (segment (start 153.43 92.18) (end 155.23 93.98) (width 0.254) (layer F.Cu) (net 2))
 (segment (start 155.23 93.98) (end 156.21 93.98) (width 0.254) (layer F.Cu) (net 2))
 (segment (start 156.2 91.45) (end 156.21 91.44) (width 0.25) (layer F.Cu) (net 1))
 (segment (start 151.31 90.18) (end 154.95 90.18) (width 0.254) (layer F.Cu) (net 1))
 (segment (start 154.95 90.18) (end 156.21 91.44) (width 0.254) (layer F.Cu) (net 1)))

